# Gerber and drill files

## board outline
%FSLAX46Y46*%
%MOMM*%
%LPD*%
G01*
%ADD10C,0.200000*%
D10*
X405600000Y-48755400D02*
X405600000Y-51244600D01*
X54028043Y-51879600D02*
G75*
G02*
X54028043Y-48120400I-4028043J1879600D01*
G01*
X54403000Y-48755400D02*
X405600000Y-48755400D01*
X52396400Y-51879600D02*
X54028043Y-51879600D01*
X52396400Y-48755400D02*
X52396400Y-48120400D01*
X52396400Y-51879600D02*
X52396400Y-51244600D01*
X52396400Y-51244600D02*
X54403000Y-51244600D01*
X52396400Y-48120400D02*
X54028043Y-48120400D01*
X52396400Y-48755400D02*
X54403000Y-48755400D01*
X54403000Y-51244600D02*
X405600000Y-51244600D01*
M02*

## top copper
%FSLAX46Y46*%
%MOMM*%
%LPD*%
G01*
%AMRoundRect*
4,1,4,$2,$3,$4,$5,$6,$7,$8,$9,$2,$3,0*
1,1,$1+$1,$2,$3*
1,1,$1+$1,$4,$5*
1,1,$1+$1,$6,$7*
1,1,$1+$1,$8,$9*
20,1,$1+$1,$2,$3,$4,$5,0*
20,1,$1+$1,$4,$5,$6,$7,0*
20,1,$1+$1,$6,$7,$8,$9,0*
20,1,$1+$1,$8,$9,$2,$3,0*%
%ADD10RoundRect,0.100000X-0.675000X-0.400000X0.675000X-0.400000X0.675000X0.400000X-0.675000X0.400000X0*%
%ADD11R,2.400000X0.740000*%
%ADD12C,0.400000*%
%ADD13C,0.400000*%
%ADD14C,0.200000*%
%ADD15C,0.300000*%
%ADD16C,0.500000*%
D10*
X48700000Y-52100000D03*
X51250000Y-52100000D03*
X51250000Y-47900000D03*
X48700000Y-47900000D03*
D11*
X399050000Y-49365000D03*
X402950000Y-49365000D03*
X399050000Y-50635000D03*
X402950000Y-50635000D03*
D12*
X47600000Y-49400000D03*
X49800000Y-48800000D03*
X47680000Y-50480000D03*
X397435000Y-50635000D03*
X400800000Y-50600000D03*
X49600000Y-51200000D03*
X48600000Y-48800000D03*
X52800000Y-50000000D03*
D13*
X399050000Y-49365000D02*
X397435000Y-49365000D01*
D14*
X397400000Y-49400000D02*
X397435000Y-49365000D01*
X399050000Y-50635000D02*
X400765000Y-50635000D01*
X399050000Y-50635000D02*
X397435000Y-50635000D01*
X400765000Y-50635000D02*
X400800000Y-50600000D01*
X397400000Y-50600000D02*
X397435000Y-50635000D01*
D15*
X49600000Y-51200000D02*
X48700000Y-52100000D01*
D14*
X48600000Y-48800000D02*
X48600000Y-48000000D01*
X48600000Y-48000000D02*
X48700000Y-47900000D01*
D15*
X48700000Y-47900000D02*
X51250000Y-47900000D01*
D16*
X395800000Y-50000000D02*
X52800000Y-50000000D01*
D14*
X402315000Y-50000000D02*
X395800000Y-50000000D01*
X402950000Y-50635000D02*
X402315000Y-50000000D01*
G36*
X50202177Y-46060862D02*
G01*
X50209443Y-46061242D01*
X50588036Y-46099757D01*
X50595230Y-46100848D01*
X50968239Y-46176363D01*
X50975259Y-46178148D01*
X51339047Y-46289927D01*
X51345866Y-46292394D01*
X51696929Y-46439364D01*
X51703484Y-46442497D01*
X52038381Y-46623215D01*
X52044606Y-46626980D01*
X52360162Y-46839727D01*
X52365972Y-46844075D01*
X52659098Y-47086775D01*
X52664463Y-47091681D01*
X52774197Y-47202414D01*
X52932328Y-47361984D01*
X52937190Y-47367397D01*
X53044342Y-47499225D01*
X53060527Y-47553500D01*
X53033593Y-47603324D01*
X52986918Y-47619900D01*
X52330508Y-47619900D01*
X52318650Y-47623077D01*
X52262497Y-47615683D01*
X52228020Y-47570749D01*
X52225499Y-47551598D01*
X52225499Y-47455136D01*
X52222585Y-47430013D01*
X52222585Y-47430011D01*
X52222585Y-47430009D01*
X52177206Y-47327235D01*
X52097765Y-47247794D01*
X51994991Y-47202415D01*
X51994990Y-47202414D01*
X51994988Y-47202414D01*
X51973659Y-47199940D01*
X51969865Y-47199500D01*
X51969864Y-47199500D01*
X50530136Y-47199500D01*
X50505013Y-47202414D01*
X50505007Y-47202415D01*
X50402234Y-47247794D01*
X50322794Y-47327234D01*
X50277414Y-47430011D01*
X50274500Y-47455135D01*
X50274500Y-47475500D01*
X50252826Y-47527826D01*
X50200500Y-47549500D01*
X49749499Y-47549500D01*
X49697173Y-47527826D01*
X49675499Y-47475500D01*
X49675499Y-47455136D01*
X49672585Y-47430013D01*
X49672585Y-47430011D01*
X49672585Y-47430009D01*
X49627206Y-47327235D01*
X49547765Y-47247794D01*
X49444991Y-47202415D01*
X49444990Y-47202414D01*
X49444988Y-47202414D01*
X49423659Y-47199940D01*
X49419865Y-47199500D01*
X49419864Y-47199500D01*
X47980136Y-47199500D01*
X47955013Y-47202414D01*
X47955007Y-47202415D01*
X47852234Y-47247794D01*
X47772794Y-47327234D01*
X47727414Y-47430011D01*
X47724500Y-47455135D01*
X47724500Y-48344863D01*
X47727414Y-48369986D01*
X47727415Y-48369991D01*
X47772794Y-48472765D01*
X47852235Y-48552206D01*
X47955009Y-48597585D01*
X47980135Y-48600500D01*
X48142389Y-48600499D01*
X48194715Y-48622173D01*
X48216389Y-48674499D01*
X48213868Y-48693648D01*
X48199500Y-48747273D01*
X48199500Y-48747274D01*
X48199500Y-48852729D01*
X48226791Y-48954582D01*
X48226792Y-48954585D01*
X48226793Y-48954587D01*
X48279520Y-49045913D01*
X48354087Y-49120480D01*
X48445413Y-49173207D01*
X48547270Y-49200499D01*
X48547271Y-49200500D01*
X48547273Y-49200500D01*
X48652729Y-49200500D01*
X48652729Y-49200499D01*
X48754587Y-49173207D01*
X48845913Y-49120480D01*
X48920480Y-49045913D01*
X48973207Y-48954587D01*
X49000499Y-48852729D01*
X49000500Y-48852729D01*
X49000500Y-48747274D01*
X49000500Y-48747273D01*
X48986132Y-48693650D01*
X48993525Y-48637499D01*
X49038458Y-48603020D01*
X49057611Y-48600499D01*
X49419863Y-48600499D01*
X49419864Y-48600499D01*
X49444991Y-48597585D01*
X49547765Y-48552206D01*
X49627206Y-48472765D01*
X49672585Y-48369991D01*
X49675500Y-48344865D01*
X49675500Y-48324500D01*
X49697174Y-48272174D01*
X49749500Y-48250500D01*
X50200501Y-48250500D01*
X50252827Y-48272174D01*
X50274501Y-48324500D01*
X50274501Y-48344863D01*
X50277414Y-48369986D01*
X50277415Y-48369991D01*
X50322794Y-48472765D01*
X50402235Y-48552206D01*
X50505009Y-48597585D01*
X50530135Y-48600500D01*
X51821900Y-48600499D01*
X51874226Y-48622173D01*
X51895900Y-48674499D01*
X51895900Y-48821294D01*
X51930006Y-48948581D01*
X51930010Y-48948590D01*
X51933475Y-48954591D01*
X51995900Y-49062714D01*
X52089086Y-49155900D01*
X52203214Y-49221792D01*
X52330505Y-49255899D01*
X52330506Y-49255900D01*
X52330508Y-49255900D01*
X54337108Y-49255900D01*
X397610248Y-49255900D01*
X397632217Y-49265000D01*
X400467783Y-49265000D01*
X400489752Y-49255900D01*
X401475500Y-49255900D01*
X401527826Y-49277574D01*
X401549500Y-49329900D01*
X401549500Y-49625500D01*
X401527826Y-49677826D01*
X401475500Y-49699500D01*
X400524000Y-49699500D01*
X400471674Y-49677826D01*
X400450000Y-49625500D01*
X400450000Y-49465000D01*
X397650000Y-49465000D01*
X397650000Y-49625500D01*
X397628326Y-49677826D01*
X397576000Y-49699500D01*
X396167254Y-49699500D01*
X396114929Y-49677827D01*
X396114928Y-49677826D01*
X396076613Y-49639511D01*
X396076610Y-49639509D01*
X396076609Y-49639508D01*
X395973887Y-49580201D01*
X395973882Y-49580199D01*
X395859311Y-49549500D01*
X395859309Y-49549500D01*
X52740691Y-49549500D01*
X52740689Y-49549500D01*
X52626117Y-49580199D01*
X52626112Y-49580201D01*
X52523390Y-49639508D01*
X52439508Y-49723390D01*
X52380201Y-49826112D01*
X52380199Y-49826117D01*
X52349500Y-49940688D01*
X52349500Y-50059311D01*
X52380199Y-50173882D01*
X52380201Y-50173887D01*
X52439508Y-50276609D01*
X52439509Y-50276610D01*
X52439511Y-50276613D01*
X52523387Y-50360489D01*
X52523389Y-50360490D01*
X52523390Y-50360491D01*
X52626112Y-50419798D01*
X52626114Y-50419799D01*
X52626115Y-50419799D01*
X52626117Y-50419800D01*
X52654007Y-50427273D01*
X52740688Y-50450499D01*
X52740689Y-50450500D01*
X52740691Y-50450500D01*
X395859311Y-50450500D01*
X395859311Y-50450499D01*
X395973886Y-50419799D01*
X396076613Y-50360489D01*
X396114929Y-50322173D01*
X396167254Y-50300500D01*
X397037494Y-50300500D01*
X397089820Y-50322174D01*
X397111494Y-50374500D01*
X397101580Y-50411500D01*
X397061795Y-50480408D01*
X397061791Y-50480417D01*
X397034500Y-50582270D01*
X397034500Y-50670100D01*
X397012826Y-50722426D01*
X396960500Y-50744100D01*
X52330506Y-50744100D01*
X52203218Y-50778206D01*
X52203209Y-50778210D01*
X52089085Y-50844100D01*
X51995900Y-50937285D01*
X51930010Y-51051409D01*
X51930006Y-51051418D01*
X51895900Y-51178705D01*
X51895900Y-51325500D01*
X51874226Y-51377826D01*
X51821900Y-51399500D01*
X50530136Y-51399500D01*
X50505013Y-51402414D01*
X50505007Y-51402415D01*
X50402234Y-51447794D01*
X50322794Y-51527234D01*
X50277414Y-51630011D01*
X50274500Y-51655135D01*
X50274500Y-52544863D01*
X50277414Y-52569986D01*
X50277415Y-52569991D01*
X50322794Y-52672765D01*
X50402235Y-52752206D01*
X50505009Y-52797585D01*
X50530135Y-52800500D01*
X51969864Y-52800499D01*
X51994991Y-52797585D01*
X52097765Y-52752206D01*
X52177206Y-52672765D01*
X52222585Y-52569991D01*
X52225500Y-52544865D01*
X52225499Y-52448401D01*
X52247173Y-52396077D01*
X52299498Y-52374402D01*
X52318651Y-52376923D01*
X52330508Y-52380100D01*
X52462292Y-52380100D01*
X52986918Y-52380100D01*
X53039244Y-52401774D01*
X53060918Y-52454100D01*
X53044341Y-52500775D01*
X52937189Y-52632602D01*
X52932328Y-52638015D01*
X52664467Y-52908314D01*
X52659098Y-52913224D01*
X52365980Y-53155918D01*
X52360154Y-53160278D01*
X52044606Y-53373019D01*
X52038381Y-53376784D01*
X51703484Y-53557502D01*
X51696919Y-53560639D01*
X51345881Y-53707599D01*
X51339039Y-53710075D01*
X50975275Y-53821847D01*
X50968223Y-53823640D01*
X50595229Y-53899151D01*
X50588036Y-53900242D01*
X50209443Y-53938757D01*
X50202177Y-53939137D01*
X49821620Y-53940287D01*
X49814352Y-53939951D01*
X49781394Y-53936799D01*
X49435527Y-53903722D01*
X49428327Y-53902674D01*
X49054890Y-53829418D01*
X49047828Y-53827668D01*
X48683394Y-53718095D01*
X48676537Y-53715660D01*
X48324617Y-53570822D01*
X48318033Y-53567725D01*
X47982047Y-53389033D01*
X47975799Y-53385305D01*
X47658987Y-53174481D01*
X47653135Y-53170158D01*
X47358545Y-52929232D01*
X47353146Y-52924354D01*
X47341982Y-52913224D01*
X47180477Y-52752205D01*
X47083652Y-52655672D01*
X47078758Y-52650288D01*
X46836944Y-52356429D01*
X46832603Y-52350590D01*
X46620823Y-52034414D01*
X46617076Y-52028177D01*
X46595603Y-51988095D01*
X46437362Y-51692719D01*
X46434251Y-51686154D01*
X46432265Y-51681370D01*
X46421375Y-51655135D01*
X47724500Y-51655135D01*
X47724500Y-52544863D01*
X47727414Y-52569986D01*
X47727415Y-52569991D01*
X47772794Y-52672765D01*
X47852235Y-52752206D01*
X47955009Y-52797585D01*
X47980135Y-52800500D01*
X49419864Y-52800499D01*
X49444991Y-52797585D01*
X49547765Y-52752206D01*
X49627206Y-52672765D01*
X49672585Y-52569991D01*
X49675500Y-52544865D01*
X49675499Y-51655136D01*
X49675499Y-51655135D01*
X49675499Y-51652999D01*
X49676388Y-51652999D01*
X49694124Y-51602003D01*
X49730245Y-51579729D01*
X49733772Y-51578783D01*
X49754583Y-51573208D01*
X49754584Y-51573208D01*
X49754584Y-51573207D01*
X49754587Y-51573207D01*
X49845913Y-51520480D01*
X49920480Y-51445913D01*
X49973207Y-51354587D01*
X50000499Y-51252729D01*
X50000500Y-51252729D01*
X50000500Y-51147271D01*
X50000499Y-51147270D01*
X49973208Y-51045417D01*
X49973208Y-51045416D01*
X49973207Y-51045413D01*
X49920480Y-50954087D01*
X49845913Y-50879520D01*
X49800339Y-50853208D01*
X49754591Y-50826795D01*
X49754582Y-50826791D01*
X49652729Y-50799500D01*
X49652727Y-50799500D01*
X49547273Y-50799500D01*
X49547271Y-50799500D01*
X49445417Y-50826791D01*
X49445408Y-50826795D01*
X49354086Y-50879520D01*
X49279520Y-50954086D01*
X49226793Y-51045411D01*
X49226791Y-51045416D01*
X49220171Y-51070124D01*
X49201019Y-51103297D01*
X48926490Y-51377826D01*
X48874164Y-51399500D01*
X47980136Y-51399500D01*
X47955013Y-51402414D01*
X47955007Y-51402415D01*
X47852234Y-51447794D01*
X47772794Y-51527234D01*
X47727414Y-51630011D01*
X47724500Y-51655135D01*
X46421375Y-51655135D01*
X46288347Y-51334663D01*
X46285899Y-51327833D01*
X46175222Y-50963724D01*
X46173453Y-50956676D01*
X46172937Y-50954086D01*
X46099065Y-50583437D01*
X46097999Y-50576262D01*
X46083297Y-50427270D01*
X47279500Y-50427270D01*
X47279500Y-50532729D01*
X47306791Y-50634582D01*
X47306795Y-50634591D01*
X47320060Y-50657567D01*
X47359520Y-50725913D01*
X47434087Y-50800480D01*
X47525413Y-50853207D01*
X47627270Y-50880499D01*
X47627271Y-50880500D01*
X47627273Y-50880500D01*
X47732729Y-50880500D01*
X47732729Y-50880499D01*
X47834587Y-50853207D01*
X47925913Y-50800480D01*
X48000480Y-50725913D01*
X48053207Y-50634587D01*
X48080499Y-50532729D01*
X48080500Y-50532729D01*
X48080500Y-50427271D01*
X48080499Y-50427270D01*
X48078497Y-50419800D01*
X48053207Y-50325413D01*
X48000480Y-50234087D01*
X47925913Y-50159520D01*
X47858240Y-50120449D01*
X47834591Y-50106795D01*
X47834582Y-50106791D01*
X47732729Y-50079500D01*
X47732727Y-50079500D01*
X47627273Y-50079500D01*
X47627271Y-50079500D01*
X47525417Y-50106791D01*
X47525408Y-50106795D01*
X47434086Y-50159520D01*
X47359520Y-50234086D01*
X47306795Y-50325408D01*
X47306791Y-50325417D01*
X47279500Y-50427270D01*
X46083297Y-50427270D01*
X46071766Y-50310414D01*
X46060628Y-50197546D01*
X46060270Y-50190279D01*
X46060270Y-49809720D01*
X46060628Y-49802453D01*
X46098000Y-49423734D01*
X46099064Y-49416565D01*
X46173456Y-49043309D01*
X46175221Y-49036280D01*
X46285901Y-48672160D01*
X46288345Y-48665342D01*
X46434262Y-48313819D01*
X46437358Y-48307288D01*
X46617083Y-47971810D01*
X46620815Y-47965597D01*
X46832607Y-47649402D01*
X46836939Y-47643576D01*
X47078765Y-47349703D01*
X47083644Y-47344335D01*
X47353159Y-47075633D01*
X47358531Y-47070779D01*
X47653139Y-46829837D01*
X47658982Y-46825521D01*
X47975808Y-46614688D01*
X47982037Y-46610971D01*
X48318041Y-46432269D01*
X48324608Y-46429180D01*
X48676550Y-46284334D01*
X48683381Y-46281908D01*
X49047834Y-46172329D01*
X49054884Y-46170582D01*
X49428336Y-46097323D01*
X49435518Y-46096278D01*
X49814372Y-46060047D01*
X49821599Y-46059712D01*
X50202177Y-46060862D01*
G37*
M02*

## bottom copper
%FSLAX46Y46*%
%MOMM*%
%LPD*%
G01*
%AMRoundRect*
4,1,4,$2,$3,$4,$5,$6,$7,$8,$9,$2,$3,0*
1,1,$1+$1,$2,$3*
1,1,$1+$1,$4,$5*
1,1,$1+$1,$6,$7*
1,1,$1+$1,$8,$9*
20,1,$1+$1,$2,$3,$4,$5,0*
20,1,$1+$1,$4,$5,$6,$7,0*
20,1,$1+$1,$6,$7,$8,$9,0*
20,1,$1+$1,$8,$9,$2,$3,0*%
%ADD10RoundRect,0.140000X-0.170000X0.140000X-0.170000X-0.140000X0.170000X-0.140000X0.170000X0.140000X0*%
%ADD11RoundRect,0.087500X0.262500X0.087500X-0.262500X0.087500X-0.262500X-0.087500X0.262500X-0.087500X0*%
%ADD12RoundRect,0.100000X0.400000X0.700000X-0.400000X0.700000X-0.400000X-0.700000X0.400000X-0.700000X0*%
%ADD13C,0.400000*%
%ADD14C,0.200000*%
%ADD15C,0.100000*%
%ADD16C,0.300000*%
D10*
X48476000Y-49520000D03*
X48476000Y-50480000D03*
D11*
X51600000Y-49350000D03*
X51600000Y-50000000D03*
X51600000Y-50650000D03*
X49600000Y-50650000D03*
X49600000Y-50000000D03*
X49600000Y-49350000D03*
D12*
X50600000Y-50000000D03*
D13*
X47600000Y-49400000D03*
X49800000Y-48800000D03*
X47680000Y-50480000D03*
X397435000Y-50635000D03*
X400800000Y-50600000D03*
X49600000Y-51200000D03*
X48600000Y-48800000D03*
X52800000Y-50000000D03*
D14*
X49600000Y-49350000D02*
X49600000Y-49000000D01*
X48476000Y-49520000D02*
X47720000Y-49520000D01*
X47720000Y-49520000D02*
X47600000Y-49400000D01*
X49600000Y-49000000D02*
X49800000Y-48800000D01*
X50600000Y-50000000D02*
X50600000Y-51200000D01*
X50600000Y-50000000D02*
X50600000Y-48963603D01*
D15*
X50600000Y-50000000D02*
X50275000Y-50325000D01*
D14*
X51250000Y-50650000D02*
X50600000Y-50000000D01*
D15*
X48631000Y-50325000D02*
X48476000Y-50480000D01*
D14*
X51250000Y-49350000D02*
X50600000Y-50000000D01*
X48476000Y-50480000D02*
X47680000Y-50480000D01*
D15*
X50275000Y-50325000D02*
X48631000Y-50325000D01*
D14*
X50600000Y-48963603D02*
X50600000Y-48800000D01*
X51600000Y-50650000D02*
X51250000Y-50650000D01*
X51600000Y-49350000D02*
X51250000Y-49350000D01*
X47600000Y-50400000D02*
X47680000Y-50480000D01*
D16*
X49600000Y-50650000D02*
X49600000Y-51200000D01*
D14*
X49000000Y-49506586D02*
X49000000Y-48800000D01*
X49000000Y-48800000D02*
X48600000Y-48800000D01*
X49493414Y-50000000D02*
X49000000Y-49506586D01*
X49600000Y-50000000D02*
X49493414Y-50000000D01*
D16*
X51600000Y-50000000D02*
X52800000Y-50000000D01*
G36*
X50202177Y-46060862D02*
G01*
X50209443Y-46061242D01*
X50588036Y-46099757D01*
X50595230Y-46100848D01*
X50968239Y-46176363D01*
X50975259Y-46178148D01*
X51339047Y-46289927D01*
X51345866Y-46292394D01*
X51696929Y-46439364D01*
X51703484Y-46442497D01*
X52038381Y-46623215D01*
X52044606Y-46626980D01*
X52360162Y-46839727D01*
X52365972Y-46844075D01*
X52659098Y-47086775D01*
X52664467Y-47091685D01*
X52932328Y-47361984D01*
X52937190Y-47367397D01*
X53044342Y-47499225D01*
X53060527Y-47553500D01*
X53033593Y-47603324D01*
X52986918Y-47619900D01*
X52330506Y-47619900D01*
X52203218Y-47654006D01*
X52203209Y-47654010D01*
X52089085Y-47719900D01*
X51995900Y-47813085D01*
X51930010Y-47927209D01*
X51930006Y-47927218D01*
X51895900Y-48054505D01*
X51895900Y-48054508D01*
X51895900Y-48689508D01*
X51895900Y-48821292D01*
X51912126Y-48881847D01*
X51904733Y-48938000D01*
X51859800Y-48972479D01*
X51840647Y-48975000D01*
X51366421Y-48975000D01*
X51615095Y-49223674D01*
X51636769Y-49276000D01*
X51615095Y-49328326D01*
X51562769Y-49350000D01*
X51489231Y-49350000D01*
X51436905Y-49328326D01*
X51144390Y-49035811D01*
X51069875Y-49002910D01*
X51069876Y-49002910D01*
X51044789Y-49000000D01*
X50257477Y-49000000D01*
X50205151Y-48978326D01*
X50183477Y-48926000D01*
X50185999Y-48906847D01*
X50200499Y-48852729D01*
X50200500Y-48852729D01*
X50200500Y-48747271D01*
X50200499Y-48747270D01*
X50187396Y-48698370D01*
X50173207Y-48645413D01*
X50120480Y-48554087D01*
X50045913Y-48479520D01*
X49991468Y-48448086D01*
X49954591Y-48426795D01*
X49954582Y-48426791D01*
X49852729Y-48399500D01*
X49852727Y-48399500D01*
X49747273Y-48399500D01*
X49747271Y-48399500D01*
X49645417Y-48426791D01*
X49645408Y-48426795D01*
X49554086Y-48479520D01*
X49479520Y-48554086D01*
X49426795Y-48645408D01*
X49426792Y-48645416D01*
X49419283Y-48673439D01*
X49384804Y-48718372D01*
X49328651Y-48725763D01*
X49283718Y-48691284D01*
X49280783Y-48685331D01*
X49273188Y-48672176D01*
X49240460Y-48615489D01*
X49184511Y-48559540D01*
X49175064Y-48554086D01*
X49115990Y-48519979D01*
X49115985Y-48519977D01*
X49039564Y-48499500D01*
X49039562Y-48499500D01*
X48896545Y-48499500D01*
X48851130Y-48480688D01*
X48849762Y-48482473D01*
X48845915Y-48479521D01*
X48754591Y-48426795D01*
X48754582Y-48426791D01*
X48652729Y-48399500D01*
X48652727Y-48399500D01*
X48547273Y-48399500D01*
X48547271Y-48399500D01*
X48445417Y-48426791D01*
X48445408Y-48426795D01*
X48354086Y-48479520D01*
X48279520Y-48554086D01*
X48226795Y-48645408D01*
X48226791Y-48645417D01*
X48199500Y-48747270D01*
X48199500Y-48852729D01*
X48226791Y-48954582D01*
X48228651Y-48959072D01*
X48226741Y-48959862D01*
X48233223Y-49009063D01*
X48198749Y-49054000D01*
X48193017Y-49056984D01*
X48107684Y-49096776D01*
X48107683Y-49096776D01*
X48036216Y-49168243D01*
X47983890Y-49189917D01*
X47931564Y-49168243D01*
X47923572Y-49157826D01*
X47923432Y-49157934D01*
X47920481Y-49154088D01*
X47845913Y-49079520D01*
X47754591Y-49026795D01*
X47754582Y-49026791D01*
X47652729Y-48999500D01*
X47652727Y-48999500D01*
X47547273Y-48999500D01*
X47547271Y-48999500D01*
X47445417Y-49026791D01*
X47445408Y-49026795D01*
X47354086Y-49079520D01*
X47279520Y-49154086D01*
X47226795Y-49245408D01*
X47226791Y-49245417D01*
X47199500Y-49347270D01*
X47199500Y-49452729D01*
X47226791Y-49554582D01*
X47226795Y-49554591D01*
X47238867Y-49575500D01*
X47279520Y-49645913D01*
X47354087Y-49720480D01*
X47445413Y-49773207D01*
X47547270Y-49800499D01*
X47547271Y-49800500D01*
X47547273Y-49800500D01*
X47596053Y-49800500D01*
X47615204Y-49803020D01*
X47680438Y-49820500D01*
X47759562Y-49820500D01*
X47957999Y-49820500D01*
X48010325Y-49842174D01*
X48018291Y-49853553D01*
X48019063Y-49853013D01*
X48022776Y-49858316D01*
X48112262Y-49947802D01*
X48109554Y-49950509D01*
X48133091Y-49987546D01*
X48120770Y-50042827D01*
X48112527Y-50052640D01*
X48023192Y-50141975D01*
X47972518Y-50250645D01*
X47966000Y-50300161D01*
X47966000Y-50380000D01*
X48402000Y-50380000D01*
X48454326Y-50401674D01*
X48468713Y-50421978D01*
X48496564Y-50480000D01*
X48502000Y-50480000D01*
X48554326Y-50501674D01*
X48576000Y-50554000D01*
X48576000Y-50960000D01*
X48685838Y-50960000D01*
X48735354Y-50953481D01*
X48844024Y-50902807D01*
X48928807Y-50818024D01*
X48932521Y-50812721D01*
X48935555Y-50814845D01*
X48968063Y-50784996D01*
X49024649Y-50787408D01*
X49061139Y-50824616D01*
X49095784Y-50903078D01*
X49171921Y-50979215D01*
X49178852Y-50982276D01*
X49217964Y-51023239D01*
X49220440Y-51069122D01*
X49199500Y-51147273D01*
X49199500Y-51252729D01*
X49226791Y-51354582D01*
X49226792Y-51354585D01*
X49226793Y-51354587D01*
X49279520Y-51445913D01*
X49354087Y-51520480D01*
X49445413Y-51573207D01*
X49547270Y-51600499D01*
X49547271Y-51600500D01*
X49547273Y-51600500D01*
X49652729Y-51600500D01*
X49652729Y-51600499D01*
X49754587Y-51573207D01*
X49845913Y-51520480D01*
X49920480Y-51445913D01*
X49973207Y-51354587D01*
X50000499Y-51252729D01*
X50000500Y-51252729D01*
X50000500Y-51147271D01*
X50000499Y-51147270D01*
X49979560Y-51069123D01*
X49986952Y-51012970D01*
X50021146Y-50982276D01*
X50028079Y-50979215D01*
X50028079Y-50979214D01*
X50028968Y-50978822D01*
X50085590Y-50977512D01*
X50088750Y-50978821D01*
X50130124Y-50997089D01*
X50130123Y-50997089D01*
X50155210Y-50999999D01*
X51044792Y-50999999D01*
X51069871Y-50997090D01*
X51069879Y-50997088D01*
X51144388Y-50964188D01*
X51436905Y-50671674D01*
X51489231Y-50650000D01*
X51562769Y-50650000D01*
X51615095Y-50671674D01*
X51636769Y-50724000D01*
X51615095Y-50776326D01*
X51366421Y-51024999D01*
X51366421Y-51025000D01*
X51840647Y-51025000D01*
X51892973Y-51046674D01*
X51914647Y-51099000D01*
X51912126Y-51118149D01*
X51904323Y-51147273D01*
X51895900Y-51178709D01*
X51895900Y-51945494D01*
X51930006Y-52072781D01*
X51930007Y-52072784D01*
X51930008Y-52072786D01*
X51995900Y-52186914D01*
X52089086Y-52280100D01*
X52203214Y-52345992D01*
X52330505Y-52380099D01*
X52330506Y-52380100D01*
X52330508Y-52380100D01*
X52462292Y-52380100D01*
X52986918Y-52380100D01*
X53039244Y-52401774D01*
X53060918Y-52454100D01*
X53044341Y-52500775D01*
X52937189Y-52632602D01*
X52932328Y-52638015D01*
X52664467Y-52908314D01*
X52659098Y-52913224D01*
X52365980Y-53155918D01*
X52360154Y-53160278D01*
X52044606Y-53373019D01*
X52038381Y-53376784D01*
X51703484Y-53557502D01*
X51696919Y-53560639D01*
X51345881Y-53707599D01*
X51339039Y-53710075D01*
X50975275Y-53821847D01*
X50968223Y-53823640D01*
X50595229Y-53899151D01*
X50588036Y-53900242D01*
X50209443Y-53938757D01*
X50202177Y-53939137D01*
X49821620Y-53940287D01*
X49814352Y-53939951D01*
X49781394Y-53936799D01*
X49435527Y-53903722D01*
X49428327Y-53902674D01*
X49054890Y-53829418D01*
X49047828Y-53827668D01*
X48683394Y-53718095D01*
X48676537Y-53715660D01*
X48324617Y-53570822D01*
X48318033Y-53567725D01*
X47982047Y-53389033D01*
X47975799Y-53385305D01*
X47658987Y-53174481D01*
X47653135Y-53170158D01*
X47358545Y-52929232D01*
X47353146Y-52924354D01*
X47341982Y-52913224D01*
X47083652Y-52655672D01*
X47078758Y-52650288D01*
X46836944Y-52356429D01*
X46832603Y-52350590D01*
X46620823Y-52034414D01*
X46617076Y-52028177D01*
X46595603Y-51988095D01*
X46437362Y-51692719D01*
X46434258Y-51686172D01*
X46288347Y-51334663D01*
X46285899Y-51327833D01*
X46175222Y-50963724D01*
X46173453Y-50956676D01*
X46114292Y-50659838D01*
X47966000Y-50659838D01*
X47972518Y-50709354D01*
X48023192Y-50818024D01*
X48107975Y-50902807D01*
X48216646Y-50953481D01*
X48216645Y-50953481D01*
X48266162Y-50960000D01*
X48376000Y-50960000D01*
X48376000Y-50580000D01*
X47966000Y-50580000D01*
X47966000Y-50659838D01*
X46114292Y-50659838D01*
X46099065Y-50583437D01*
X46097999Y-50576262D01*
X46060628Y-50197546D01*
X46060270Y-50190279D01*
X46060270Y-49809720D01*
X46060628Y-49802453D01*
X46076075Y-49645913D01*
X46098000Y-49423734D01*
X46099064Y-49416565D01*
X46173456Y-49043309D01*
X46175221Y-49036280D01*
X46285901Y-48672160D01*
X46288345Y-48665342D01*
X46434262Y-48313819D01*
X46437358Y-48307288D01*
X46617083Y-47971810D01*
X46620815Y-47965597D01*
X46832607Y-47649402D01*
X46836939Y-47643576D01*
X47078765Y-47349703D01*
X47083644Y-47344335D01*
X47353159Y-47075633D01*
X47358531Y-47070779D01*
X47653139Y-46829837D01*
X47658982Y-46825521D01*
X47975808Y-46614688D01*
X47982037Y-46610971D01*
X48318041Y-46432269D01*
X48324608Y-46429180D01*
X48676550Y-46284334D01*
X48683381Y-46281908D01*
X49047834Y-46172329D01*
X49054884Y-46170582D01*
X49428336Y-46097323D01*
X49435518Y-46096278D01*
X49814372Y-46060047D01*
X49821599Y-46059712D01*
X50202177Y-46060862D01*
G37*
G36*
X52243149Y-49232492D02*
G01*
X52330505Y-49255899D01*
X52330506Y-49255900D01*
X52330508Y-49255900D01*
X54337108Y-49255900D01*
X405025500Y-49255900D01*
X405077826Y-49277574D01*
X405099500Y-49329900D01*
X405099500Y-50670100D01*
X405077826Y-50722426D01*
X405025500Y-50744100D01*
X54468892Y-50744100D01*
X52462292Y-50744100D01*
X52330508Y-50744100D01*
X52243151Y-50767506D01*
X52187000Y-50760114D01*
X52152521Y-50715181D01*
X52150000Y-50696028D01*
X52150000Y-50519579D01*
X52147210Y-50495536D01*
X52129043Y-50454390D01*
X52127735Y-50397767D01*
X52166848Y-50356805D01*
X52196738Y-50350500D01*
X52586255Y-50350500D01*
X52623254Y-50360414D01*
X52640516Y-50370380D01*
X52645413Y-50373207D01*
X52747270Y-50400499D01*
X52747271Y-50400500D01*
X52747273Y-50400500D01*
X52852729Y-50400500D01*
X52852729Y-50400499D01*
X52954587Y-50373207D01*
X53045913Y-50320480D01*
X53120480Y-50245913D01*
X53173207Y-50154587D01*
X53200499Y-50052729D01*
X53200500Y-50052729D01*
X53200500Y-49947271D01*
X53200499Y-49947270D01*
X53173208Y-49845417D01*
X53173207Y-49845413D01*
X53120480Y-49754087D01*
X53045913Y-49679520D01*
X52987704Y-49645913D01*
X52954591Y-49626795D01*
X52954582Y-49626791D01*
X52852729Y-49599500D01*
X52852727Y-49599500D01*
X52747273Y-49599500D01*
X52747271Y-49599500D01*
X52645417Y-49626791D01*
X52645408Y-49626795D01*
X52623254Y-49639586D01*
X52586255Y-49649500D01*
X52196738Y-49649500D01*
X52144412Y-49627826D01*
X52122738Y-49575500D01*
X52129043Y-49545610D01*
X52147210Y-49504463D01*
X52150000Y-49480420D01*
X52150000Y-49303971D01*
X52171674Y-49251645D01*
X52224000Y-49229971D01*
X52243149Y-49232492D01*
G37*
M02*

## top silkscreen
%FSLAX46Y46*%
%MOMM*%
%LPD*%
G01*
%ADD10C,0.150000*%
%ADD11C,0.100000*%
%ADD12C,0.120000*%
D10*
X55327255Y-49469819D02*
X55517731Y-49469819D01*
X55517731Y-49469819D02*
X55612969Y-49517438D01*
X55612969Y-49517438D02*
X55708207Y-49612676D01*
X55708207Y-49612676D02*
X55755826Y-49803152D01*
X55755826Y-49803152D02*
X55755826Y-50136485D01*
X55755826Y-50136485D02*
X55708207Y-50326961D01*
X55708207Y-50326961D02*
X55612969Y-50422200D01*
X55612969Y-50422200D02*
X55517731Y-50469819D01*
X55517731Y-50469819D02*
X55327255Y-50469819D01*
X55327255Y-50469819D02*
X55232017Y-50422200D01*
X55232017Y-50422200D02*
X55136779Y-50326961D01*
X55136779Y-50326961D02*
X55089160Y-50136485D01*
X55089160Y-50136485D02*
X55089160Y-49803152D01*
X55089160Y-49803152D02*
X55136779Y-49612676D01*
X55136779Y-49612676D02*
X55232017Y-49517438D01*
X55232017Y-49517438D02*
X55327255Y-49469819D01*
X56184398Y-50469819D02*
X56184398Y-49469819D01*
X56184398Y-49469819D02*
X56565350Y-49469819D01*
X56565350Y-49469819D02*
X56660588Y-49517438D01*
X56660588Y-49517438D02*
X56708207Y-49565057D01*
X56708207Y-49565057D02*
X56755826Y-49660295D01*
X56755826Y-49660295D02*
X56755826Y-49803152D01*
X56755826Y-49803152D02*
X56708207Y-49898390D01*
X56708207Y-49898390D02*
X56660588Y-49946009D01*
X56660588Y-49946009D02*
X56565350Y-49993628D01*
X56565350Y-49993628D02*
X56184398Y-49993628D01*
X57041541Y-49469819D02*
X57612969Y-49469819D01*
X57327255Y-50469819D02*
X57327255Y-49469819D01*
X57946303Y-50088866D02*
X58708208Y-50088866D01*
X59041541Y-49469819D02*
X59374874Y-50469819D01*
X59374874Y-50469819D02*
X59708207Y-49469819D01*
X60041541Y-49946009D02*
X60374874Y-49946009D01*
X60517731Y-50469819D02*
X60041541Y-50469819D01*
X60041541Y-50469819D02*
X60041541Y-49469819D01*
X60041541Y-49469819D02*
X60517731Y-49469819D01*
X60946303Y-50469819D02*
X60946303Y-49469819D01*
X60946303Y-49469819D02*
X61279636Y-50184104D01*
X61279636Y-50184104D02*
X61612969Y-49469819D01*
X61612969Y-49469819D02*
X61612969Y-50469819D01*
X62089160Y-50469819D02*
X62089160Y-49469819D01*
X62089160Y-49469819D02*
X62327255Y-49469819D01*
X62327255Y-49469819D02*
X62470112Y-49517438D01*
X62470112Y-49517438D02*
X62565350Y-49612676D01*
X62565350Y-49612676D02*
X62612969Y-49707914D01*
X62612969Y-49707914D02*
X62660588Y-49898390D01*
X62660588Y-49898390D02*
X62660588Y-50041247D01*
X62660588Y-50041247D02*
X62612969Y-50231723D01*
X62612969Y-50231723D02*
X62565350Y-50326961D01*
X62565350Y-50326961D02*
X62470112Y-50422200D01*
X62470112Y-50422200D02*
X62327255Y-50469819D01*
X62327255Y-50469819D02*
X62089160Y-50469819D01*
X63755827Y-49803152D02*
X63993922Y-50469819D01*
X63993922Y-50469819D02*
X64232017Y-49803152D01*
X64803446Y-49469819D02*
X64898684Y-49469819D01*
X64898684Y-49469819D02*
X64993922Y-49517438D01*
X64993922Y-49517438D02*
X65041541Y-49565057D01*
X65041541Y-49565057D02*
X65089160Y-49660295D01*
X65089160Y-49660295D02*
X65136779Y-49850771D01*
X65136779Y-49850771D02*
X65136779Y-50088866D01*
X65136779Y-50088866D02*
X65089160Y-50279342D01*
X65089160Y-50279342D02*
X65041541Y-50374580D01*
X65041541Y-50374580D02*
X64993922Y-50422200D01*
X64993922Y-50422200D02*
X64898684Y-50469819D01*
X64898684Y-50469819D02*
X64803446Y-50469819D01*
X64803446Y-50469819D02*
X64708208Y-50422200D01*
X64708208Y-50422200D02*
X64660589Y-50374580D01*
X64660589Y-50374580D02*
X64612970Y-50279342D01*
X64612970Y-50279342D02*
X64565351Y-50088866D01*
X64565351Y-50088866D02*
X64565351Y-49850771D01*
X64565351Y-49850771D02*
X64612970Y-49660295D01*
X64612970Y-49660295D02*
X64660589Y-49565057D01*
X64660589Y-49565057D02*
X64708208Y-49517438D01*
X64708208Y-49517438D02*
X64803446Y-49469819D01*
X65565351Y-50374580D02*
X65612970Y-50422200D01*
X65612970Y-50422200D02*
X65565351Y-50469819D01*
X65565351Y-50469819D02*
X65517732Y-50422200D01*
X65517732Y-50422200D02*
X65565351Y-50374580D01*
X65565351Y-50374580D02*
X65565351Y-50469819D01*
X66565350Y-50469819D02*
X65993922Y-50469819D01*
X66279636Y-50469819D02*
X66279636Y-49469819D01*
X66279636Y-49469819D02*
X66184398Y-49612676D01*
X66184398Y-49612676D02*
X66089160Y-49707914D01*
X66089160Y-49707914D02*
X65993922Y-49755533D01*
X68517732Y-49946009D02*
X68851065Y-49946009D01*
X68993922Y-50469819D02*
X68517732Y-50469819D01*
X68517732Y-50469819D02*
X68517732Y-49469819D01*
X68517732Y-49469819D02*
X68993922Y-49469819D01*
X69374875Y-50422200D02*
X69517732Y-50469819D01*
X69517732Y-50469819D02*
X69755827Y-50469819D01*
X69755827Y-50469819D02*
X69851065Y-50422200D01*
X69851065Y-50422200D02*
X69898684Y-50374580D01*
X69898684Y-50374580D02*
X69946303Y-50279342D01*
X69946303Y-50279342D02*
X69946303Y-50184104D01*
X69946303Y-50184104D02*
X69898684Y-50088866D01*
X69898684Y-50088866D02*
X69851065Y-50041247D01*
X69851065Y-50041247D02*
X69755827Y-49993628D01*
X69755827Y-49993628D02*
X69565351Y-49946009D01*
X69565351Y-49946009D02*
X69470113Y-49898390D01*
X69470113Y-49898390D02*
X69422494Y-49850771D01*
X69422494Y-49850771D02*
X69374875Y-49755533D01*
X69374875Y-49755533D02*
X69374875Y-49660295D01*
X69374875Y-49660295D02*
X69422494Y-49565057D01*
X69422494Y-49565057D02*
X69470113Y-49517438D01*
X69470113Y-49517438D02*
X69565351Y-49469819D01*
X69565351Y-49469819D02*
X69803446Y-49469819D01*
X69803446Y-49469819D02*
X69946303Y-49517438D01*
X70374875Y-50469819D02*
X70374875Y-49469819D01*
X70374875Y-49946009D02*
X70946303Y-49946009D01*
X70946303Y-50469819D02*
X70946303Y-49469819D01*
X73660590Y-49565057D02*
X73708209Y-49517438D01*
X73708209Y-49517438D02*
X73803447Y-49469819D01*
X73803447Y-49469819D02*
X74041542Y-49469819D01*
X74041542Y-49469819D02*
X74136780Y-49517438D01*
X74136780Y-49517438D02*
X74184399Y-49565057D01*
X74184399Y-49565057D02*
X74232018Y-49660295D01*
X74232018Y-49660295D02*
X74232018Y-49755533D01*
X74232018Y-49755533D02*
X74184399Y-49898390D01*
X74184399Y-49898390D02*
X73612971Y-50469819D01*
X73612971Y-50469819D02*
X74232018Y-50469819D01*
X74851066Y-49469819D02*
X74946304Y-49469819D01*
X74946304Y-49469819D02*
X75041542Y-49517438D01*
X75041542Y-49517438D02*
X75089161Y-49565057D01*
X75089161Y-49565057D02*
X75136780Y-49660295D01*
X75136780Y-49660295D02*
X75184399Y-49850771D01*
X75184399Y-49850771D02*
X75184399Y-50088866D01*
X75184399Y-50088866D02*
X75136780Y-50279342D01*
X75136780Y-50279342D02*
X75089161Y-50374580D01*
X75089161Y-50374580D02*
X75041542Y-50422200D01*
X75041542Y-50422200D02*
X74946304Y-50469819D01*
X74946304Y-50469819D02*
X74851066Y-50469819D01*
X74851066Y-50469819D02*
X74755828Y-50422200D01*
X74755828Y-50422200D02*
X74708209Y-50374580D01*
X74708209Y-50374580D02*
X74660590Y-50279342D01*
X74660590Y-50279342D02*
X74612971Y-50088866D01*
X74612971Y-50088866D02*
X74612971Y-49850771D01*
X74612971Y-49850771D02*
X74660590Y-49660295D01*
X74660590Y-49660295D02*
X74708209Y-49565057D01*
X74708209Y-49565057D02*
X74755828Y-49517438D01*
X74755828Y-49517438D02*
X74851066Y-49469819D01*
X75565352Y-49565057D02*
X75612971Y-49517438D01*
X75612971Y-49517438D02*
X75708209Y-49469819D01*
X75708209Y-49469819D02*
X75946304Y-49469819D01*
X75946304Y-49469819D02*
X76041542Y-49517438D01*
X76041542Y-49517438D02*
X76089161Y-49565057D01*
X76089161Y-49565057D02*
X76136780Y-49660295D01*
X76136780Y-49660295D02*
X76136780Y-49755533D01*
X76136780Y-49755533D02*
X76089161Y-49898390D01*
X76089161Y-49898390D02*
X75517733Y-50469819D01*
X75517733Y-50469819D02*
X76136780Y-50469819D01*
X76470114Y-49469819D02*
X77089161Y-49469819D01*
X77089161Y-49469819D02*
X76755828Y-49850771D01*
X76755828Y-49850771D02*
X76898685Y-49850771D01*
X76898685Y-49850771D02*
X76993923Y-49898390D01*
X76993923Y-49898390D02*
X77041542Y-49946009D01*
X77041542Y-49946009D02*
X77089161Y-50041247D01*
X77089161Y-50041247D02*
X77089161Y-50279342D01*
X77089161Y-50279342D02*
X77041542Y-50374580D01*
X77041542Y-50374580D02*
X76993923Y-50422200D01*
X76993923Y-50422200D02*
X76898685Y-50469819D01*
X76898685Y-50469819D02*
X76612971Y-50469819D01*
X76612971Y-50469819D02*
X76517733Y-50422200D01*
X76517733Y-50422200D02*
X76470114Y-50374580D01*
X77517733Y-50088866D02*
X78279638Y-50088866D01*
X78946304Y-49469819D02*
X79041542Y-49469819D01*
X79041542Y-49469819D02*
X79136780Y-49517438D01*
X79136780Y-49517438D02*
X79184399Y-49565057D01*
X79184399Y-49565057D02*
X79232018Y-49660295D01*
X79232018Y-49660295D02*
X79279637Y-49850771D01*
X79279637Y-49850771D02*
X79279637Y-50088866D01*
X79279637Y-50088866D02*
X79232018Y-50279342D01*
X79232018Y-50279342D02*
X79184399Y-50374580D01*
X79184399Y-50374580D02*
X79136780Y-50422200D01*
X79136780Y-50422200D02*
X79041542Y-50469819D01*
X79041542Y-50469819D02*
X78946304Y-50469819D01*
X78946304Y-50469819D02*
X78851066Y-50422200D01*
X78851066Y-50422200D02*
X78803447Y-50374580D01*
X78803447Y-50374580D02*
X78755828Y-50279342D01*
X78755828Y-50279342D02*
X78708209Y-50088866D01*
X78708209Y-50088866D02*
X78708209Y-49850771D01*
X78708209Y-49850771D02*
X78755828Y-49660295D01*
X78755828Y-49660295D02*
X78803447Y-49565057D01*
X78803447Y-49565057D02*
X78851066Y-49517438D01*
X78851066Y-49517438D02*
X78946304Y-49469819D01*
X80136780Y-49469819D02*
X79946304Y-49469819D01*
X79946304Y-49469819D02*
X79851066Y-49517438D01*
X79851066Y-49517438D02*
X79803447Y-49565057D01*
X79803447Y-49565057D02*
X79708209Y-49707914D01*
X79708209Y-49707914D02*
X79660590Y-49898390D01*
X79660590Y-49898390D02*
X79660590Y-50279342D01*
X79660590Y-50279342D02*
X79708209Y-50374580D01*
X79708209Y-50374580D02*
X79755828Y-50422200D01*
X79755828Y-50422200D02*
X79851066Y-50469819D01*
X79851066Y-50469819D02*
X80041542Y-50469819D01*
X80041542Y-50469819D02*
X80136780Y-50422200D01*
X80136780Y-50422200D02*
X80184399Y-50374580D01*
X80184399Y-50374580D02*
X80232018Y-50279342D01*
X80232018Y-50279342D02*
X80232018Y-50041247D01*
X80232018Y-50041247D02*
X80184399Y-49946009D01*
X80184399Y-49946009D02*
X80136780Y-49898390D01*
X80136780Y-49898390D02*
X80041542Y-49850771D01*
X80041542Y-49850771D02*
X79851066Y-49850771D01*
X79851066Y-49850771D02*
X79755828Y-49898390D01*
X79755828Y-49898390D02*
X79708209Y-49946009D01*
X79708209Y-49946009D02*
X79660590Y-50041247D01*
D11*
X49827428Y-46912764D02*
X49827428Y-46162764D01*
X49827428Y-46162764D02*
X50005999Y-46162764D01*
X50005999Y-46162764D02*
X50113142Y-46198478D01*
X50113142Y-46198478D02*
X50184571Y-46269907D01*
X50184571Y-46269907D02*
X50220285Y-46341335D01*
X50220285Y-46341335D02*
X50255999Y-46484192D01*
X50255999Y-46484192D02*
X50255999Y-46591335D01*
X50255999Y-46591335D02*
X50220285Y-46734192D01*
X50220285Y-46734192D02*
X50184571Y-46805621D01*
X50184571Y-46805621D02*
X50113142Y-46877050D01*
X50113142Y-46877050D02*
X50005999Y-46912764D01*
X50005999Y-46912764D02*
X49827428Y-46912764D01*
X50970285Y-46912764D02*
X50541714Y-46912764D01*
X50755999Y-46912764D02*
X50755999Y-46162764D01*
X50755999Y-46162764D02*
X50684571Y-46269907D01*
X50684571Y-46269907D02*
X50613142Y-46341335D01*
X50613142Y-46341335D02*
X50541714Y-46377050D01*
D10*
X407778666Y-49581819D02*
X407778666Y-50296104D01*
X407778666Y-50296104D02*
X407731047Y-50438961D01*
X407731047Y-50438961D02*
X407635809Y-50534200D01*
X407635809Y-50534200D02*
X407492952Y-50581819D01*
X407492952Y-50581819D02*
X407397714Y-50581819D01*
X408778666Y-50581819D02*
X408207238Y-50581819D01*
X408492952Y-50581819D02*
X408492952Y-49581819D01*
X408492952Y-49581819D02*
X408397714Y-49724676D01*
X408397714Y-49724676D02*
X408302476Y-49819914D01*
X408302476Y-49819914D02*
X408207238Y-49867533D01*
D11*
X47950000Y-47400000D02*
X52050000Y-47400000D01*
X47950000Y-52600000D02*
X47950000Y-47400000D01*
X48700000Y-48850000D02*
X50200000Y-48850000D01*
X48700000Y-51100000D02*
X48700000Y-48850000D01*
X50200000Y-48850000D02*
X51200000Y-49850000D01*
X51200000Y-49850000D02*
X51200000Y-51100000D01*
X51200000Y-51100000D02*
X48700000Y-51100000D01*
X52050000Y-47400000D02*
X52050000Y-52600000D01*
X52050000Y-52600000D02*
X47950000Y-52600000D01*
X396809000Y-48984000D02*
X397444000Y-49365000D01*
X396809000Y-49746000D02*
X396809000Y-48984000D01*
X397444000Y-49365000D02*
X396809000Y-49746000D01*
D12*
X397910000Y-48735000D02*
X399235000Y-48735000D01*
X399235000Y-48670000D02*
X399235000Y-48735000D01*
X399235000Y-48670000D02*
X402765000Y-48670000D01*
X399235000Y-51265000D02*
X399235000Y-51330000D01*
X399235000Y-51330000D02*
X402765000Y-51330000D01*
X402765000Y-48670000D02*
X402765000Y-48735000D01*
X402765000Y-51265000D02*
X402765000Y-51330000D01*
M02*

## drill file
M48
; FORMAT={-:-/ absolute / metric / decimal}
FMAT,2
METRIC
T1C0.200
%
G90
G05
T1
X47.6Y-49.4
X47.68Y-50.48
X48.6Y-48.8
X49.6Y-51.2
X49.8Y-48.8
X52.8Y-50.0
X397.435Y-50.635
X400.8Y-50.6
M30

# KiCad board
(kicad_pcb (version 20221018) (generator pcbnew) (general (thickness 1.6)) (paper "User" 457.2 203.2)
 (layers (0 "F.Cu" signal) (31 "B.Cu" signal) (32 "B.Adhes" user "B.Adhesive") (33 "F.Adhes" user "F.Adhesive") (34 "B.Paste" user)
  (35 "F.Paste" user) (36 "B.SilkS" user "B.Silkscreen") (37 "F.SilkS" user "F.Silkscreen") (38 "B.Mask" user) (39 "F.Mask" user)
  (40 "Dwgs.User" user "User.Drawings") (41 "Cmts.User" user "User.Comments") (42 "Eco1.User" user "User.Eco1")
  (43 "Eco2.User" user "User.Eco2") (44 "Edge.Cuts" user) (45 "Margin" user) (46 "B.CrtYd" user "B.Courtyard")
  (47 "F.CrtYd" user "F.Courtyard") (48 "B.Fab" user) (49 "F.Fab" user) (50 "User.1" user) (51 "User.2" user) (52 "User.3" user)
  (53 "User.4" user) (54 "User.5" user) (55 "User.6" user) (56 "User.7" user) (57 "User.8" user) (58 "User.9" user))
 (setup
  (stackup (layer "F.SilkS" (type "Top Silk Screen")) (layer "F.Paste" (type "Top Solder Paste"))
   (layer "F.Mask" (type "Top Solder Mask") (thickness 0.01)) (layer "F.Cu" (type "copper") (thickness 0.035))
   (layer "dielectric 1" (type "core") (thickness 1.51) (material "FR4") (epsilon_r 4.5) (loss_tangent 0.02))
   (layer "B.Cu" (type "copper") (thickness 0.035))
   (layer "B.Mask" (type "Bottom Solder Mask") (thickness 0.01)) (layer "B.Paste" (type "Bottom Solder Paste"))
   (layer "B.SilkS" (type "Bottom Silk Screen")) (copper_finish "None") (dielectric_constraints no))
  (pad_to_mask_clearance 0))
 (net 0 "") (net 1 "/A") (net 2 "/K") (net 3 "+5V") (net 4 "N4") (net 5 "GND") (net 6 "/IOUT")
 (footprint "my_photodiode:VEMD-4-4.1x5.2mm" (layer "F.Cu") (at 48.7 52.1)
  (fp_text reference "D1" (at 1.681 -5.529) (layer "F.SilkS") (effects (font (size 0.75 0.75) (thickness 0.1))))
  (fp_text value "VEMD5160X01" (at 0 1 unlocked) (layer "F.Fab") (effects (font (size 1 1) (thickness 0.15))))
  (fp_line (start -0.75 -4.7) (end 3.35 -4.7) (stroke (width 0.1) (type default)) (layer "F.SilkS"))
  (fp_line (start -0.75 0.5) (end -0.75 -4.7) (stroke (width 0.1) (type default)) (layer "F.SilkS"))
  (fp_line (start 0 -3.25) (end 1.5 -3.25) (stroke (width 0.1) (type default)) (layer "F.SilkS"))
  (fp_line (start 0 -1) (end 0 -3.25) (stroke (width 0.1) (type default)) (layer "F.SilkS"))
  (fp_line (start 1.5 -3.25) (end 2.5 -2.25) (stroke (width 0.1) (type default)) (layer "F.SilkS"))
  (fp_line (start 2.5 -2.25) (end 2.5 -1) (stroke (width 0.1) (type default)) (layer "F.SilkS"))
  (fp_line (start 2.5 -1) (end 0 -1) (stroke (width 0.1) (type default)) (layer "F.SilkS"))
  (fp_line (start 3.35 -4.7) (end 3.35 0.5) (stroke (width 0.1) (type default)) (layer "F.SilkS"))
  (fp_line (start 3.35 0.5) (end -0.75 0.5) (stroke (width 0.1) (type default)) (layer "F.SilkS"))
  (pad "1" smd roundrect (at 0 0) (size 1.55 1) (layers "F.Cu" "F.Paste" "F.Mask") (roundrect_rratio 0.1) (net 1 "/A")
   (thermal_bridge_angle 45))
  (pad "2" smd roundrect (at 2.55 0) (size 1.55 1) (layers "F.Cu" "F.Paste" "F.Mask") (roundrect_rratio 0.1) (thermal_bridge_angle 45))
  (pad "3" smd roundrect (at 2.55 -4.2) (size 1.55 1) (layers "F.Cu" "F.Paste" "F.Mask") (roundrect_rratio 0.1) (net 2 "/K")
   (thermal_bridge_angle 45))
  (pad "4" smd roundrect (at 0 -4.2) (size 1.55 1) (layers "F.Cu" "F.Paste" "F.Mask") (roundrect_rratio 0.1) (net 2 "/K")
   (thermal_bridge_angle 45)))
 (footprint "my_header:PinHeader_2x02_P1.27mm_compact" (layer "F.Cu") (at 401 50)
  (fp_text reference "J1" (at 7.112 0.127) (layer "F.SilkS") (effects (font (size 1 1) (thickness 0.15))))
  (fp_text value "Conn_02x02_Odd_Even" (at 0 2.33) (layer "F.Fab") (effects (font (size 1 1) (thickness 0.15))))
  (fp_line (start -4.191 -1.016) (end -3.556 -0.635) (stroke (width 0.1) (type default)) (layer "F.SilkS"))
  (fp_line (start -4.191 -0.254) (end -4.191 -1.016) (stroke (width 0.1) (type default)) (layer "F.SilkS"))
  (fp_line (start -3.556 -0.635) (end -4.191 -0.254) (stroke (width 0.1) (type default)) (layer "F.SilkS"))
  (fp_line (start -3.09 -1.265) (end -1.765 -1.265) (stroke (width 0.12) (type solid)) (layer "F.SilkS"))
  (fp_line (start -1.765 -1.33) (end -1.765 -1.265) (stroke (width 0.12) (type solid)) (layer "F.SilkS"))
  (fp_line (start -1.765 -1.33) (end 1.765 -1.33) (stroke (width 0.12) (type solid)) (layer "F.SilkS"))
  (fp_line (start -1.765 1.265) (end -1.765 1.33) (stroke (width 0.12) (type solid)) (layer "F.SilkS"))
  (fp_line (start -1.765 1.33) (end 1.765 1.33) (stroke (width 0.12) (type solid)) (layer "F.SilkS"))
  (fp_line (start 1.765 -1.33) (end 1.765 -1.265) (stroke (width 0.12) (type solid)) (layer "F.SilkS"))
  (fp_line (start 1.765 1.265) (end 1.765 1.33) (stroke (width 0.12) (type solid)) (layer "F.SilkS"))
  (pad "1" smd rect (at -1.95 -0.635) (size 2.4 0.74) (layers "F.Cu" "F.Paste" "F.Mask") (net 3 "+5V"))
  (pad "2" smd rect (at 1.95 -0.635) (size 2.4 0.74) (layers "F.Cu" "F.Paste" "F.Mask") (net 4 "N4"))
  (pad "3" smd rect (at -1.95 0.635) (size 2.4 0.74) (layers "F.Cu" "F.Paste" "F.Mask") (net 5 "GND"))
  (pad "4" smd rect (at 1.95 0.635) (size 2.4 0.74) (layers "F.Cu" "F.Paste" "F.Mask") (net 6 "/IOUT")))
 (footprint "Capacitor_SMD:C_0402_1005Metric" (layer "B.Cu") (at 48.476 50 -90)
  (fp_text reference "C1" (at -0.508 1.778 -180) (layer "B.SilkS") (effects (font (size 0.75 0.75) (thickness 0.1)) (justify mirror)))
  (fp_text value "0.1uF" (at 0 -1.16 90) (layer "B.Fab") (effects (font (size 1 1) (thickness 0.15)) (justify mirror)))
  (pad "1" smd roundrect (at -0.48 0 270) (size 0.56 0.62) (layers "B.Cu" "B.Paste" "B.Mask") (roundrect_rratio 0.25) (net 3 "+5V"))
  (pad "2" smd roundrect (at 0.48 0 270) (size 0.56 0.62) (layers "B.Cu" "B.Paste" "B.Mask") (roundrect_rratio 0.25) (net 5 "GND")))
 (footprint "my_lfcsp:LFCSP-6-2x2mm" (layer "B.Cu") (at 51.6 49.35 180)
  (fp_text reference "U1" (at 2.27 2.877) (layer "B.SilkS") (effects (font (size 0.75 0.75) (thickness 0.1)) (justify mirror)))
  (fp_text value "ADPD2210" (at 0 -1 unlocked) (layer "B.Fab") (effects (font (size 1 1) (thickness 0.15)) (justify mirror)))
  (pad "1" smd roundrect (at 0 0 180) (size 0.7 0.35) (layers "B.Cu" "B.Paste" "B.Mask") (roundrect_rratio 0.25) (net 5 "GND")
   (thermal_bridge_angle 45))
  (pad "2" smd roundrect (at 0 -0.65 180) (size 0.7 0.35) (layers "B.Cu" "B.Paste" "B.Mask") (roundrect_rratio 0.25) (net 6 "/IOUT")
   (thermal_bridge_angle 45))
  (pad "3" smd roundrect (at 0 -1.3 180) (size 0.7 0.35) (layers "B.Cu" "B.Paste" "B.Mask") (roundrect_rratio 0.25) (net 5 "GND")
   (thermal_bridge_angle 45))
  (pad "4" smd roundrect (at 2 -1.3 180) (size 0.7 0.35) (layers "B.Cu" "B.Paste" "B.Mask") (roundrect_rratio 0.25) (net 1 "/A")
   (thermal_bridge_angle 45))
  (pad "5" smd roundrect (at 2 -0.65 180) (size 0.7 0.35) (layers "B.Cu" "B.Paste" "B.Mask") (roundrect_rratio 0.25) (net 2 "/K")
   (thermal_bridge_angle 45))
  (pad "6" smd roundrect (at 2 0 180) (size 0.7 0.35) (layers "B.Cu" "B.Paste" "B.Mask") (roundrect_rratio 0.25) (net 3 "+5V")
   (thermal_bridge_angle 45))
  (pad "7" smd roundrect (at 1 -0.65 180) (size 1 1.6) (layers "B.Cu" "B.Paste" "B.Mask") (roundrect_rratio 0.1) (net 5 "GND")
   (thermal_bridge_angle 45)))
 (gr_line (start 405.6 48.7554) (end 405.6 51.2446) (stroke (width 0.2) (type solid)) (layer "Edge.Cuts"))
 (gr_arc (start 54.028043 51.8796) (mid 45.555 50) (end 54.028043 48.1204) (stroke (width 0.2) (type solid)) (layer "Edge.Cuts"))
 (gr_line (start 54.403 48.7554) (end 405.6 48.7554) (stroke (width 0.2) (type solid)) (layer "Edge.Cuts"))
 (gr_line (start 52.3964 51.8796) (end 54.028043 51.8796) (stroke (width 0.2) (type solid)) (layer "Edge.Cuts"))
 (gr_line (start 52.3964 48.7554) (end 52.3964 48.1204) (stroke (width 0.2) (type solid)) (layer "Edge.Cuts"))
 (gr_line (start 52.3964 51.8796) (end 52.3964 51.2446) (stroke (width 0.2) (type solid)) (layer "Edge.Cuts"))
 (gr_line (start 52.3964 51.2446) (end 54.403 51.2446) (stroke (width 0.2) (type solid)) (layer "Edge.Cuts"))
 (gr_line (start 52.3964 48.1204) (end 54.028043 48.1204) (stroke (width 0.2) (type solid)) (layer "Edge.Cuts"))
 (gr_line (start 52.3964 48.7554) (end 54.403 48.7554) (stroke (width 0.2) (type solid)) (layer "Edge.Cuts"))
 (gr_line (start 54.403 51.2446) (end 405.6 51.2446) (stroke (width 0.2) (type solid)) (layer "Edge.Cuts"))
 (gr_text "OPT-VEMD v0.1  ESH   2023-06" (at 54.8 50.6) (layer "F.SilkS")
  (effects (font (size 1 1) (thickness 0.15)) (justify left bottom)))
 (segment (start 399.05 49.365) (end 397.435 49.365) (width 0.4) (layer "F.Cu") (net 3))
 (segment (start 397.4 49.4) (end 397.435 49.365) (width 0.2) (layer "F.Cu") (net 3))
 (via (at 47.6 49.4) (size 0.4) (drill 0.2) (layers "F.Cu" "B.Cu") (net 3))
 (via (at 49.8 48.8) (size 0.4) (drill 0.2) (layers "F.Cu" "B.Cu") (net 3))
 (segment (start 49.6 49.35) (end 49.6 49) (width 0.2) (layer "B.Cu") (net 3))
 (segment (start 48.476 49.52) (end 47.72 49.52) (width 0.2) (layer "B.Cu") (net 3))
 (segment (start 47.72 49.52) (end 47.6 49.4) (width 0.2) (layer "B.Cu") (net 3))
 (segment (start 49.6 49) (end 49.8 48.8) (width 0.2) (layer "B.Cu") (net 3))
 (segment (start 399.05 50.635) (end 400.765 50.635) (width 0.2) (layer "F.Cu") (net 5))
 (segment (start 399.05 50.635) (end 397.435 50.635) (width 0.2) (layer "F.Cu") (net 5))
 (segment (start 400.765 50.635) (end 400.8 50.6) (width 0.2) (layer "F.Cu") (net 5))
 (segment (start 397.4 50.6) (end 397.435 50.635) (width 0.2) (layer "F.Cu") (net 5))
 (via (at 47.68 50.48) (size 0.4) (drill 0.2) (layers "F.Cu" "B.Cu") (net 5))
 (via (at 397.435 50.635) (size 0.4) (drill 0.2) (layers "F.Cu" "B.Cu") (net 5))
 (via (at 400.8 50.6) (size 0.4) (drill 0.2) (layers "F.Cu" "B.Cu") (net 5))
 (segment (start 50.6 50) (end 50.6 51.2) (width 0.2) (layer "B.Cu") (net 5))
 (segment (start 50.6 50) (end 50.6 48.963603) (width 0.2) (layer "B.Cu") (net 5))
 (segment (start 50.6 50) (end 50.275 50.325) (width 0.1) (layer "B.Cu") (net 5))
 (segment (start 51.25 50.65) (end 50.6 50) (width 0.2) (layer "B.Cu") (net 5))
 (segment (start 48.631 50.325) (end 48.476 50.48) (width 0.1) (layer "B.Cu") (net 5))
 (segment (start 51.25 49.35) (end 50.6 50) (width 0.2) (layer "B.Cu") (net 5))
 (segment (start 48.476 50.48) (end 47.68 50.48) (width 0.2) (layer "B.Cu") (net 5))
 (segment (start 50.275 50.325) (end 48.631 50.325) (width 0.1) (layer "B.Cu") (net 5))
 (segment (start 50.6 48.963603) (end 50.6 48.8) (width 0.2) (layer "B.Cu") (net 5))
 (segment (start 51.6 50.65) (end 51.25 50.65) (width 0.2) (layer "B.Cu") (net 5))
 (segment (start 51.6 49.35) (end 51.25 49.35) (width 0.2) (layer "B.Cu") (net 5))
 (segment (start 47.6 50.4) (end 47.68 50.48) (width 0.2) (layer "B.Cu") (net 5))
 (segment (start 49.6 51.2) (end 48.7 52.1) (width 0.3) (layer "F.Cu") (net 1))
 (via (at 49.6 51.2) (size 0.4) (drill 0.2) (layers "F.Cu" "B.Cu") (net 1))
 (segment (start 49.6 50.65) (end 49.6 51.2) (width 0.3) (layer "B.Cu") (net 1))
 (segment (start 48.6 48.8) (end 48.6 48) (width 0.2) (layer "F.Cu") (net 2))
 (segment (start 48.6 48) (end 48.7 47.9) (width 0.2) (layer "F.Cu") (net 2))
 (segment (start 48.7 47.9) (end 51.25 47.9) (width 0.3) (layer "F.Cu") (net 2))
 (via (at 48.6 48.8) (size 0.4) (drill 0.2) (layers "F.Cu" "B.Cu") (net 2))
 (segment (start 49 49.506586) (end 49 48.8) (width 0.2) (layer "B.Cu") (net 2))
 (segment (start 49 48.8) (end 48.6 48.8) (width 0.2) (layer "B.Cu") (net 2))
 (segment (start 49.493414 50) (end 49 49.506586) (width 0.2) (layer "B.Cu") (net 2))
 (segment (start 49.6 50) (end 49.493414 50) (width 0.2) (layer "B.Cu") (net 2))
 (segment (start 395.8 50) (end 52.8 50) (width 0.5) (layer "F.Cu") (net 6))
 (segment (start 402.315 50) (end 395.8 50) (width 0.2) (layer "F.Cu") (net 6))
 (segment (start 402.95 50.635) (end 402.315 50) (width 0.2) (layer "F.Cu") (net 6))
 (via (at 52.8 50) (size 0.4) (drill 0.2) (layers "F.Cu" "B.Cu") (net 6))
 (segment (start 51.6 50) (end 52.8 50) (width 0.3) (layer "B.Cu") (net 6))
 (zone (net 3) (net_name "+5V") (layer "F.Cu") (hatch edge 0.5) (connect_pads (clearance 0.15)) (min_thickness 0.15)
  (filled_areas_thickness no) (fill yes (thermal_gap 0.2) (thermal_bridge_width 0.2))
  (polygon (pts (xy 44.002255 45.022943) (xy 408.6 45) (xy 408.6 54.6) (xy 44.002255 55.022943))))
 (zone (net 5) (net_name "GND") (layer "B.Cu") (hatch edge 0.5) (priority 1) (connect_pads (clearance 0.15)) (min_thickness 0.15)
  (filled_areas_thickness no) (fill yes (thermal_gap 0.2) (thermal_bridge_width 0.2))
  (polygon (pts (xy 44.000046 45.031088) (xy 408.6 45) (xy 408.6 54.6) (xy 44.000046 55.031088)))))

